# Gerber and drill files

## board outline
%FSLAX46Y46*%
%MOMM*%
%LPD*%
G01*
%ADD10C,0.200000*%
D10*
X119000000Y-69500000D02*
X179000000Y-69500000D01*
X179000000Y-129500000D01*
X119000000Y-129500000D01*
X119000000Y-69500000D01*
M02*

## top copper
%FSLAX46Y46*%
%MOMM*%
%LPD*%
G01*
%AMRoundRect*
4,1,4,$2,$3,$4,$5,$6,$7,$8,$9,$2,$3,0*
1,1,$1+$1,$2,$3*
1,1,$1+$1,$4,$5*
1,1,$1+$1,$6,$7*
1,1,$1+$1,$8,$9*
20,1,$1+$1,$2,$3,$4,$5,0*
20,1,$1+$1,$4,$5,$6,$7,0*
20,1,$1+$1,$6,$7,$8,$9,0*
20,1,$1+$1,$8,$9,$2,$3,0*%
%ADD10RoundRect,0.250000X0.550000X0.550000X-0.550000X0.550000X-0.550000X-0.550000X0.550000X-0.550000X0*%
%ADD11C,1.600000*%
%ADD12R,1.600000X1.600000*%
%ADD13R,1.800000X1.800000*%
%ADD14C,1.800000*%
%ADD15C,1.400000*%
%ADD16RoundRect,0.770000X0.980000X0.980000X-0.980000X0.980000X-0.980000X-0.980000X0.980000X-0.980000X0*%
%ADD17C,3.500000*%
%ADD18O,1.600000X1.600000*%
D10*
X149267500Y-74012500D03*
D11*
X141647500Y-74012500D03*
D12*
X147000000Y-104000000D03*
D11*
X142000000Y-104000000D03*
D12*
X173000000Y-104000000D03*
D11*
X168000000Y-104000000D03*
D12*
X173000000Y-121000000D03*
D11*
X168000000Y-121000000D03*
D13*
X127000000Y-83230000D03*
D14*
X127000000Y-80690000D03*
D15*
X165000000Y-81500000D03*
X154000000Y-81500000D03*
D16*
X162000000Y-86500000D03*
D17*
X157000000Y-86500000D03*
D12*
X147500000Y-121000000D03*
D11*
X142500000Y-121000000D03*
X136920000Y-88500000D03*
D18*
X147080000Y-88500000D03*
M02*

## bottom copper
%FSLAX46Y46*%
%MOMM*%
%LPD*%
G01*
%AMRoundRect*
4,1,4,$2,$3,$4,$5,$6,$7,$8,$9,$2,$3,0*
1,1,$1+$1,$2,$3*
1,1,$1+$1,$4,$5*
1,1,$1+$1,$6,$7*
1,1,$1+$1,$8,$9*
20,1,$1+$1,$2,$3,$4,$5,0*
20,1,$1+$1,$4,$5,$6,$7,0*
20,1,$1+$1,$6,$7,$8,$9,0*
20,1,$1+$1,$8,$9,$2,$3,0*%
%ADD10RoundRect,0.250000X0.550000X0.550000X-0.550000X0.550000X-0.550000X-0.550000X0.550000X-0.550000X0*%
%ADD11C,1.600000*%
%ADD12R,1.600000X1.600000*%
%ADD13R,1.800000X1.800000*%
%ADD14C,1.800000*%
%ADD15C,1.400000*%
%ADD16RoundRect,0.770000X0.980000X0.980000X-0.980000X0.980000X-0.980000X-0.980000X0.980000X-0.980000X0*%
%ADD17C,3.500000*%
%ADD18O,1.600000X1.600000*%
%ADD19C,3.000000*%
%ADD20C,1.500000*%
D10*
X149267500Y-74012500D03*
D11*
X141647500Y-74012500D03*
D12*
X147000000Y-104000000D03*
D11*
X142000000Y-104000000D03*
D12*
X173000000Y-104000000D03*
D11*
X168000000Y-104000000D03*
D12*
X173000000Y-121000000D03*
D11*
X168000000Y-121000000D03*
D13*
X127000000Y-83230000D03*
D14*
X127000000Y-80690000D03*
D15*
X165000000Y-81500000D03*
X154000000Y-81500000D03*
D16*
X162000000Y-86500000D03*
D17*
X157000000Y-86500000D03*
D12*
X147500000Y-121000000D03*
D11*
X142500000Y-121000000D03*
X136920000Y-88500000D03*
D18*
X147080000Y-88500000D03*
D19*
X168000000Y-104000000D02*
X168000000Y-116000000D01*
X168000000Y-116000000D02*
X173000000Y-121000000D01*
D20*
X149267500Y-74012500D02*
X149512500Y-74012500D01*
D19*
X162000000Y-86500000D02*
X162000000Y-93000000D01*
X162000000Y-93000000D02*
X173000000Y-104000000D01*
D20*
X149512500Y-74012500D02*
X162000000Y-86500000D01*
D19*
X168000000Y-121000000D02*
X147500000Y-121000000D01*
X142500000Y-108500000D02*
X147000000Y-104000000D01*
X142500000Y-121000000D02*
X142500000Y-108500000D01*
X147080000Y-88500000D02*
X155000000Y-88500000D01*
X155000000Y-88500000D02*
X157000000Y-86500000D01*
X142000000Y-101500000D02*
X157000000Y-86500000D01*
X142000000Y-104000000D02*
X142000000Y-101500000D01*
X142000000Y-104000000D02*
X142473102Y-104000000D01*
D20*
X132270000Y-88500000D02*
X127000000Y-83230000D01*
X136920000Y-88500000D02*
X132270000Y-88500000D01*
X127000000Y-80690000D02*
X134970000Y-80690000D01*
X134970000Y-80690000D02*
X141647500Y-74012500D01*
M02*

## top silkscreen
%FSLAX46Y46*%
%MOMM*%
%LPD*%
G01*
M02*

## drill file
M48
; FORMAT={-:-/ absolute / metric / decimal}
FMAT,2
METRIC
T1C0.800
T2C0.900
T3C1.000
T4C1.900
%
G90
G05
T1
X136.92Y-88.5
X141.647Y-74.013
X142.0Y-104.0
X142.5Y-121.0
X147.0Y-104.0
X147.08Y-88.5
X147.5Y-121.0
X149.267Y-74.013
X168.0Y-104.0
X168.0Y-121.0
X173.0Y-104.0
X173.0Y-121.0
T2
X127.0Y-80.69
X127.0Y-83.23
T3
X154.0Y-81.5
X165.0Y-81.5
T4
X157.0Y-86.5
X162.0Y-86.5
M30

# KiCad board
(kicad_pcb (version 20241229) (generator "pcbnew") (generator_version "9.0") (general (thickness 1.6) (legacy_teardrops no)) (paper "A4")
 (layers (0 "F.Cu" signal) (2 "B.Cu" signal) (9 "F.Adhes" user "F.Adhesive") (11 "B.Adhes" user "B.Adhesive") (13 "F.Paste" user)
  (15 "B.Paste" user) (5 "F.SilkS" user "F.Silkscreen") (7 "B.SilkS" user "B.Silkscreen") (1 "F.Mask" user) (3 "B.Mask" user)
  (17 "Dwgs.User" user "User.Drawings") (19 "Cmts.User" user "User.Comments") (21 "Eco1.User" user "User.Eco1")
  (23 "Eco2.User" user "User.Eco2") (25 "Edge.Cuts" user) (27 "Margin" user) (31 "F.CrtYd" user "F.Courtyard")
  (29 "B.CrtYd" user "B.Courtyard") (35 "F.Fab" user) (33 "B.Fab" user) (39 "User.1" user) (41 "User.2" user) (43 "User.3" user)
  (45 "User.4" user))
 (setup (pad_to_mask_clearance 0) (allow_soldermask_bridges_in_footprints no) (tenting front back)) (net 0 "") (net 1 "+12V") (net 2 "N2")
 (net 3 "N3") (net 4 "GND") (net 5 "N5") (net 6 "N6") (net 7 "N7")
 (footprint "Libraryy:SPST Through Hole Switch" (layer "B.Cu") (at 149.2675 74.0125 180)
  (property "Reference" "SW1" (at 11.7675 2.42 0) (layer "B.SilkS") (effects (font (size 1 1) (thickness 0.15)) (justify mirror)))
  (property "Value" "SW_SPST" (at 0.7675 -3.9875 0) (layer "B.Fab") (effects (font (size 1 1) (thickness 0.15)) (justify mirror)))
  (pad "1" thru_hole roundrect (at 0 0 180) (size 1.6 1.6) (drill 0.8) (layers "*.Cu" "*.Mask") (remove_unused_layers no)
   (roundrect_rratio 0.15625) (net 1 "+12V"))
  (pad "2" thru_hole circle (at 7.62 0 180) (size 1.6 1.6) (drill 0.8) (layers "*.Cu" "*.Mask") (remove_unused_layers no) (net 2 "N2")))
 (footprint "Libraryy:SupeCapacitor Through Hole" (layer "B.Cu") (at 147 104 180)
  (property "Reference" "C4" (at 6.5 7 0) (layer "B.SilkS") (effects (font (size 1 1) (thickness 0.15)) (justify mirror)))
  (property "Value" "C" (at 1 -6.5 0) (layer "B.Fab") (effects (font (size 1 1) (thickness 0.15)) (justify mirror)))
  (pad "1" thru_hole rect (at 0 0 180) (size 1.6 1.6) (drill 0.8) (layers "*.Cu" "*.Mask") (remove_unused_layers no) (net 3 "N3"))
  (pad "2" thru_hole circle (at 5 0 180) (size 1.6 1.6) (drill 0.8) (layers "*.Cu" "*.Mask") (remove_unused_layers no) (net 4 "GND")))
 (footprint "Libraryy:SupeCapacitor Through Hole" (layer "B.Cu") (at 173 104 180)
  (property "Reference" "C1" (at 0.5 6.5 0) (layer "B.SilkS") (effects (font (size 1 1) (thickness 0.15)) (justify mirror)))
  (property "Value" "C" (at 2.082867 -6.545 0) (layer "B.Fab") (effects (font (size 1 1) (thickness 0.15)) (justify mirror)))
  (pad "1" thru_hole rect (at 0 0 180) (size 1.6 1.6) (drill 0.8) (layers "*.Cu" "*.Mask") (remove_unused_layers no) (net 1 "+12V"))
  (pad "2" thru_hole circle (at 5 0 180) (size 1.6 1.6) (drill 0.8) (layers "*.Cu" "*.Mask") (remove_unused_layers no) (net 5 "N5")))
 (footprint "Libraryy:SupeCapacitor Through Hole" (layer "B.Cu") (at 173 121 180)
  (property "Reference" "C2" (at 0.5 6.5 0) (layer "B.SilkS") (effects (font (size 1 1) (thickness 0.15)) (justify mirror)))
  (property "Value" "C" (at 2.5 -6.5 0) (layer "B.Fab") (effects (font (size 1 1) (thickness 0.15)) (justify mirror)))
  (pad "1" thru_hole rect (at 0 0 180) (size 1.6 1.6) (drill 0.8) (layers "*.Cu" "*.Mask") (remove_unused_layers no) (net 5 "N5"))
  (pad "2" thru_hole circle (at 5 0 180) (size 1.6 1.6) (drill 0.8) (layers "*.Cu" "*.Mask") (remove_unused_layers no) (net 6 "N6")))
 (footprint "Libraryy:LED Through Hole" (layer "B.Cu") (at 127 83.23 90)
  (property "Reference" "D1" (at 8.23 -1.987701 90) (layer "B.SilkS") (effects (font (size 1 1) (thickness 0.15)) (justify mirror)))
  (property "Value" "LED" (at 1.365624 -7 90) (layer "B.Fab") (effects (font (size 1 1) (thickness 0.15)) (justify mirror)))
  (pad "1" thru_hole rect (at 0 0 90) (size 1.8 1.8) (drill 0.9) (layers "*.Cu" "*.Mask") (remove_unused_layers no) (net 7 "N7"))
  (pad "2" thru_hole circle (at 2.54 0 90) (size 1.8 1.8) (drill 0.9) (layers "*.Cu" "*.Mask") (remove_unused_layers no) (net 2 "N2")))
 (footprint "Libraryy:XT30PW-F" (layer "B.Cu") (at 162 86.5 180)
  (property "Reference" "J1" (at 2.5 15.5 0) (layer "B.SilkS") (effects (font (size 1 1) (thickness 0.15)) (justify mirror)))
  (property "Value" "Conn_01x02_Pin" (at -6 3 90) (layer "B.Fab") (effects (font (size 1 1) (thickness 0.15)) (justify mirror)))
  (pad "" thru_hole circle (at -3 5 90) (size 1.4 1.4) (drill 1) (layers "*.Cu" "*.Mask") (remove_unused_layers no))
  (pad "" thru_hole circle (at 8 5 180) (size 1.4 1.4) (drill 1) (layers "*.Cu" "*.Mask") (remove_unused_layers no))
  (pad "1" thru_hole roundrect (at 0 0 180) (size 3.5 3.5) (drill 1.9) (layers "*.Cu" "*.Mask") (remove_unused_layers no)
   (roundrect_rratio 0.22) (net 1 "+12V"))
  (pad "2" thru_hole circle (at 5 0 180) (size 3.5 3.5) (drill 1.9) (layers "*.Cu" "*.Mask") (remove_unused_layers no) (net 4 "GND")))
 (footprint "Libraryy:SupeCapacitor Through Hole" (layer "B.Cu") (at 147.5 121 180)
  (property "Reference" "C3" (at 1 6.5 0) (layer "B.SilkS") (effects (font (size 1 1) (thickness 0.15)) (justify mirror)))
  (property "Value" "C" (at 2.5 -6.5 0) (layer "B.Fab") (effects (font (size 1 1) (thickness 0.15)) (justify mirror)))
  (pad "1" thru_hole rect (at 0 0 180) (size 1.6 1.6) (drill 0.8) (layers "*.Cu" "*.Mask") (remove_unused_layers no) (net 6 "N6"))
  (pad "2" thru_hole circle (at 5 0 180) (size 1.6 1.6) (drill 0.8) (layers "*.Cu" "*.Mask") (remove_unused_layers no) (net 3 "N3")))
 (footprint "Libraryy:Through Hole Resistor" (layer "B.Cu") (at 136.92 88.5)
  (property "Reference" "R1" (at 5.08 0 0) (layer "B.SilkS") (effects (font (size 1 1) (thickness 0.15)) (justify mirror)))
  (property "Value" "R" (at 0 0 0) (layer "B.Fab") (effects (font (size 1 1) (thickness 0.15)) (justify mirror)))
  (pad "1" thru_hole circle (at 0 0) (size 1.6 1.6) (drill 0.8) (layers "*.Cu" "*.Mask") (remove_unused_layers no) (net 7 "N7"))
  (pad "2" thru_hole oval (at 10.16 0) (size 1.6 1.6) (drill 0.8) (layers "*.Cu" "*.Mask") (remove_unused_layers no) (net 4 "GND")))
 (gr_rect (start 119 69.5) (end 179 129.5) (stroke (width 0.2) (type solid)) (fill no) (layer "Edge.Cuts"))
 (segment (start 168 104) (end 168 116) (width 3) (layer "B.Cu") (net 5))
 (segment (start 168 116) (end 173 121) (width 3) (layer "B.Cu") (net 5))
 (segment (start 149.2675 74.0125) (end 149.5125 74.0125) (width 1.5) (layer "B.Cu") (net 1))
 (segment (start 162 86.5) (end 162 93) (width 3) (layer "B.Cu") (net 1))
 (segment (start 162 93) (end 173 104) (width 3) (layer "B.Cu") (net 1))
 (segment (start 149.5125 74.0125) (end 162 86.5) (width 1.5) (layer "B.Cu") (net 1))
 (segment (start 168 121) (end 147.5 121) (width 3) (layer "B.Cu") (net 6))
 (segment (start 142.5 108.5) (end 147 104) (width 3) (layer "B.Cu") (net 3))
 (segment (start 142.5 121) (end 142.5 108.5) (width 3) (layer "B.Cu") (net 3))
 (segment (start 147.08 88.5) (end 155 88.5) (width 3) (layer "B.Cu") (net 4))
 (segment (start 155 88.5) (end 157 86.5) (width 3) (layer "B.Cu") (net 4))
 (segment (start 142 101.5) (end 157 86.5) (width 3) (layer "B.Cu") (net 4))
 (segment (start 142 104) (end 142 101.5) (width 3) (layer "B.Cu") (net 4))
 (segment (start 142 104) (end 142.473102 104) (width 3) (layer "B.Cu") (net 4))
 (segment (start 132.27 88.5) (end 127 83.23) (width 1.5) (layer "B.Cu") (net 7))
 (segment (start 136.92 88.5) (end 132.27 88.5) (width 1.5) (layer "B.Cu") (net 7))
 (segment (start 127 80.69) (end 134.97 80.69) (width 1.5) (layer "B.Cu") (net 2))
 (segment (start 134.97 80.69) (end 141.6475 74.0125) (width 1.5) (layer "B.Cu") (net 2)))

